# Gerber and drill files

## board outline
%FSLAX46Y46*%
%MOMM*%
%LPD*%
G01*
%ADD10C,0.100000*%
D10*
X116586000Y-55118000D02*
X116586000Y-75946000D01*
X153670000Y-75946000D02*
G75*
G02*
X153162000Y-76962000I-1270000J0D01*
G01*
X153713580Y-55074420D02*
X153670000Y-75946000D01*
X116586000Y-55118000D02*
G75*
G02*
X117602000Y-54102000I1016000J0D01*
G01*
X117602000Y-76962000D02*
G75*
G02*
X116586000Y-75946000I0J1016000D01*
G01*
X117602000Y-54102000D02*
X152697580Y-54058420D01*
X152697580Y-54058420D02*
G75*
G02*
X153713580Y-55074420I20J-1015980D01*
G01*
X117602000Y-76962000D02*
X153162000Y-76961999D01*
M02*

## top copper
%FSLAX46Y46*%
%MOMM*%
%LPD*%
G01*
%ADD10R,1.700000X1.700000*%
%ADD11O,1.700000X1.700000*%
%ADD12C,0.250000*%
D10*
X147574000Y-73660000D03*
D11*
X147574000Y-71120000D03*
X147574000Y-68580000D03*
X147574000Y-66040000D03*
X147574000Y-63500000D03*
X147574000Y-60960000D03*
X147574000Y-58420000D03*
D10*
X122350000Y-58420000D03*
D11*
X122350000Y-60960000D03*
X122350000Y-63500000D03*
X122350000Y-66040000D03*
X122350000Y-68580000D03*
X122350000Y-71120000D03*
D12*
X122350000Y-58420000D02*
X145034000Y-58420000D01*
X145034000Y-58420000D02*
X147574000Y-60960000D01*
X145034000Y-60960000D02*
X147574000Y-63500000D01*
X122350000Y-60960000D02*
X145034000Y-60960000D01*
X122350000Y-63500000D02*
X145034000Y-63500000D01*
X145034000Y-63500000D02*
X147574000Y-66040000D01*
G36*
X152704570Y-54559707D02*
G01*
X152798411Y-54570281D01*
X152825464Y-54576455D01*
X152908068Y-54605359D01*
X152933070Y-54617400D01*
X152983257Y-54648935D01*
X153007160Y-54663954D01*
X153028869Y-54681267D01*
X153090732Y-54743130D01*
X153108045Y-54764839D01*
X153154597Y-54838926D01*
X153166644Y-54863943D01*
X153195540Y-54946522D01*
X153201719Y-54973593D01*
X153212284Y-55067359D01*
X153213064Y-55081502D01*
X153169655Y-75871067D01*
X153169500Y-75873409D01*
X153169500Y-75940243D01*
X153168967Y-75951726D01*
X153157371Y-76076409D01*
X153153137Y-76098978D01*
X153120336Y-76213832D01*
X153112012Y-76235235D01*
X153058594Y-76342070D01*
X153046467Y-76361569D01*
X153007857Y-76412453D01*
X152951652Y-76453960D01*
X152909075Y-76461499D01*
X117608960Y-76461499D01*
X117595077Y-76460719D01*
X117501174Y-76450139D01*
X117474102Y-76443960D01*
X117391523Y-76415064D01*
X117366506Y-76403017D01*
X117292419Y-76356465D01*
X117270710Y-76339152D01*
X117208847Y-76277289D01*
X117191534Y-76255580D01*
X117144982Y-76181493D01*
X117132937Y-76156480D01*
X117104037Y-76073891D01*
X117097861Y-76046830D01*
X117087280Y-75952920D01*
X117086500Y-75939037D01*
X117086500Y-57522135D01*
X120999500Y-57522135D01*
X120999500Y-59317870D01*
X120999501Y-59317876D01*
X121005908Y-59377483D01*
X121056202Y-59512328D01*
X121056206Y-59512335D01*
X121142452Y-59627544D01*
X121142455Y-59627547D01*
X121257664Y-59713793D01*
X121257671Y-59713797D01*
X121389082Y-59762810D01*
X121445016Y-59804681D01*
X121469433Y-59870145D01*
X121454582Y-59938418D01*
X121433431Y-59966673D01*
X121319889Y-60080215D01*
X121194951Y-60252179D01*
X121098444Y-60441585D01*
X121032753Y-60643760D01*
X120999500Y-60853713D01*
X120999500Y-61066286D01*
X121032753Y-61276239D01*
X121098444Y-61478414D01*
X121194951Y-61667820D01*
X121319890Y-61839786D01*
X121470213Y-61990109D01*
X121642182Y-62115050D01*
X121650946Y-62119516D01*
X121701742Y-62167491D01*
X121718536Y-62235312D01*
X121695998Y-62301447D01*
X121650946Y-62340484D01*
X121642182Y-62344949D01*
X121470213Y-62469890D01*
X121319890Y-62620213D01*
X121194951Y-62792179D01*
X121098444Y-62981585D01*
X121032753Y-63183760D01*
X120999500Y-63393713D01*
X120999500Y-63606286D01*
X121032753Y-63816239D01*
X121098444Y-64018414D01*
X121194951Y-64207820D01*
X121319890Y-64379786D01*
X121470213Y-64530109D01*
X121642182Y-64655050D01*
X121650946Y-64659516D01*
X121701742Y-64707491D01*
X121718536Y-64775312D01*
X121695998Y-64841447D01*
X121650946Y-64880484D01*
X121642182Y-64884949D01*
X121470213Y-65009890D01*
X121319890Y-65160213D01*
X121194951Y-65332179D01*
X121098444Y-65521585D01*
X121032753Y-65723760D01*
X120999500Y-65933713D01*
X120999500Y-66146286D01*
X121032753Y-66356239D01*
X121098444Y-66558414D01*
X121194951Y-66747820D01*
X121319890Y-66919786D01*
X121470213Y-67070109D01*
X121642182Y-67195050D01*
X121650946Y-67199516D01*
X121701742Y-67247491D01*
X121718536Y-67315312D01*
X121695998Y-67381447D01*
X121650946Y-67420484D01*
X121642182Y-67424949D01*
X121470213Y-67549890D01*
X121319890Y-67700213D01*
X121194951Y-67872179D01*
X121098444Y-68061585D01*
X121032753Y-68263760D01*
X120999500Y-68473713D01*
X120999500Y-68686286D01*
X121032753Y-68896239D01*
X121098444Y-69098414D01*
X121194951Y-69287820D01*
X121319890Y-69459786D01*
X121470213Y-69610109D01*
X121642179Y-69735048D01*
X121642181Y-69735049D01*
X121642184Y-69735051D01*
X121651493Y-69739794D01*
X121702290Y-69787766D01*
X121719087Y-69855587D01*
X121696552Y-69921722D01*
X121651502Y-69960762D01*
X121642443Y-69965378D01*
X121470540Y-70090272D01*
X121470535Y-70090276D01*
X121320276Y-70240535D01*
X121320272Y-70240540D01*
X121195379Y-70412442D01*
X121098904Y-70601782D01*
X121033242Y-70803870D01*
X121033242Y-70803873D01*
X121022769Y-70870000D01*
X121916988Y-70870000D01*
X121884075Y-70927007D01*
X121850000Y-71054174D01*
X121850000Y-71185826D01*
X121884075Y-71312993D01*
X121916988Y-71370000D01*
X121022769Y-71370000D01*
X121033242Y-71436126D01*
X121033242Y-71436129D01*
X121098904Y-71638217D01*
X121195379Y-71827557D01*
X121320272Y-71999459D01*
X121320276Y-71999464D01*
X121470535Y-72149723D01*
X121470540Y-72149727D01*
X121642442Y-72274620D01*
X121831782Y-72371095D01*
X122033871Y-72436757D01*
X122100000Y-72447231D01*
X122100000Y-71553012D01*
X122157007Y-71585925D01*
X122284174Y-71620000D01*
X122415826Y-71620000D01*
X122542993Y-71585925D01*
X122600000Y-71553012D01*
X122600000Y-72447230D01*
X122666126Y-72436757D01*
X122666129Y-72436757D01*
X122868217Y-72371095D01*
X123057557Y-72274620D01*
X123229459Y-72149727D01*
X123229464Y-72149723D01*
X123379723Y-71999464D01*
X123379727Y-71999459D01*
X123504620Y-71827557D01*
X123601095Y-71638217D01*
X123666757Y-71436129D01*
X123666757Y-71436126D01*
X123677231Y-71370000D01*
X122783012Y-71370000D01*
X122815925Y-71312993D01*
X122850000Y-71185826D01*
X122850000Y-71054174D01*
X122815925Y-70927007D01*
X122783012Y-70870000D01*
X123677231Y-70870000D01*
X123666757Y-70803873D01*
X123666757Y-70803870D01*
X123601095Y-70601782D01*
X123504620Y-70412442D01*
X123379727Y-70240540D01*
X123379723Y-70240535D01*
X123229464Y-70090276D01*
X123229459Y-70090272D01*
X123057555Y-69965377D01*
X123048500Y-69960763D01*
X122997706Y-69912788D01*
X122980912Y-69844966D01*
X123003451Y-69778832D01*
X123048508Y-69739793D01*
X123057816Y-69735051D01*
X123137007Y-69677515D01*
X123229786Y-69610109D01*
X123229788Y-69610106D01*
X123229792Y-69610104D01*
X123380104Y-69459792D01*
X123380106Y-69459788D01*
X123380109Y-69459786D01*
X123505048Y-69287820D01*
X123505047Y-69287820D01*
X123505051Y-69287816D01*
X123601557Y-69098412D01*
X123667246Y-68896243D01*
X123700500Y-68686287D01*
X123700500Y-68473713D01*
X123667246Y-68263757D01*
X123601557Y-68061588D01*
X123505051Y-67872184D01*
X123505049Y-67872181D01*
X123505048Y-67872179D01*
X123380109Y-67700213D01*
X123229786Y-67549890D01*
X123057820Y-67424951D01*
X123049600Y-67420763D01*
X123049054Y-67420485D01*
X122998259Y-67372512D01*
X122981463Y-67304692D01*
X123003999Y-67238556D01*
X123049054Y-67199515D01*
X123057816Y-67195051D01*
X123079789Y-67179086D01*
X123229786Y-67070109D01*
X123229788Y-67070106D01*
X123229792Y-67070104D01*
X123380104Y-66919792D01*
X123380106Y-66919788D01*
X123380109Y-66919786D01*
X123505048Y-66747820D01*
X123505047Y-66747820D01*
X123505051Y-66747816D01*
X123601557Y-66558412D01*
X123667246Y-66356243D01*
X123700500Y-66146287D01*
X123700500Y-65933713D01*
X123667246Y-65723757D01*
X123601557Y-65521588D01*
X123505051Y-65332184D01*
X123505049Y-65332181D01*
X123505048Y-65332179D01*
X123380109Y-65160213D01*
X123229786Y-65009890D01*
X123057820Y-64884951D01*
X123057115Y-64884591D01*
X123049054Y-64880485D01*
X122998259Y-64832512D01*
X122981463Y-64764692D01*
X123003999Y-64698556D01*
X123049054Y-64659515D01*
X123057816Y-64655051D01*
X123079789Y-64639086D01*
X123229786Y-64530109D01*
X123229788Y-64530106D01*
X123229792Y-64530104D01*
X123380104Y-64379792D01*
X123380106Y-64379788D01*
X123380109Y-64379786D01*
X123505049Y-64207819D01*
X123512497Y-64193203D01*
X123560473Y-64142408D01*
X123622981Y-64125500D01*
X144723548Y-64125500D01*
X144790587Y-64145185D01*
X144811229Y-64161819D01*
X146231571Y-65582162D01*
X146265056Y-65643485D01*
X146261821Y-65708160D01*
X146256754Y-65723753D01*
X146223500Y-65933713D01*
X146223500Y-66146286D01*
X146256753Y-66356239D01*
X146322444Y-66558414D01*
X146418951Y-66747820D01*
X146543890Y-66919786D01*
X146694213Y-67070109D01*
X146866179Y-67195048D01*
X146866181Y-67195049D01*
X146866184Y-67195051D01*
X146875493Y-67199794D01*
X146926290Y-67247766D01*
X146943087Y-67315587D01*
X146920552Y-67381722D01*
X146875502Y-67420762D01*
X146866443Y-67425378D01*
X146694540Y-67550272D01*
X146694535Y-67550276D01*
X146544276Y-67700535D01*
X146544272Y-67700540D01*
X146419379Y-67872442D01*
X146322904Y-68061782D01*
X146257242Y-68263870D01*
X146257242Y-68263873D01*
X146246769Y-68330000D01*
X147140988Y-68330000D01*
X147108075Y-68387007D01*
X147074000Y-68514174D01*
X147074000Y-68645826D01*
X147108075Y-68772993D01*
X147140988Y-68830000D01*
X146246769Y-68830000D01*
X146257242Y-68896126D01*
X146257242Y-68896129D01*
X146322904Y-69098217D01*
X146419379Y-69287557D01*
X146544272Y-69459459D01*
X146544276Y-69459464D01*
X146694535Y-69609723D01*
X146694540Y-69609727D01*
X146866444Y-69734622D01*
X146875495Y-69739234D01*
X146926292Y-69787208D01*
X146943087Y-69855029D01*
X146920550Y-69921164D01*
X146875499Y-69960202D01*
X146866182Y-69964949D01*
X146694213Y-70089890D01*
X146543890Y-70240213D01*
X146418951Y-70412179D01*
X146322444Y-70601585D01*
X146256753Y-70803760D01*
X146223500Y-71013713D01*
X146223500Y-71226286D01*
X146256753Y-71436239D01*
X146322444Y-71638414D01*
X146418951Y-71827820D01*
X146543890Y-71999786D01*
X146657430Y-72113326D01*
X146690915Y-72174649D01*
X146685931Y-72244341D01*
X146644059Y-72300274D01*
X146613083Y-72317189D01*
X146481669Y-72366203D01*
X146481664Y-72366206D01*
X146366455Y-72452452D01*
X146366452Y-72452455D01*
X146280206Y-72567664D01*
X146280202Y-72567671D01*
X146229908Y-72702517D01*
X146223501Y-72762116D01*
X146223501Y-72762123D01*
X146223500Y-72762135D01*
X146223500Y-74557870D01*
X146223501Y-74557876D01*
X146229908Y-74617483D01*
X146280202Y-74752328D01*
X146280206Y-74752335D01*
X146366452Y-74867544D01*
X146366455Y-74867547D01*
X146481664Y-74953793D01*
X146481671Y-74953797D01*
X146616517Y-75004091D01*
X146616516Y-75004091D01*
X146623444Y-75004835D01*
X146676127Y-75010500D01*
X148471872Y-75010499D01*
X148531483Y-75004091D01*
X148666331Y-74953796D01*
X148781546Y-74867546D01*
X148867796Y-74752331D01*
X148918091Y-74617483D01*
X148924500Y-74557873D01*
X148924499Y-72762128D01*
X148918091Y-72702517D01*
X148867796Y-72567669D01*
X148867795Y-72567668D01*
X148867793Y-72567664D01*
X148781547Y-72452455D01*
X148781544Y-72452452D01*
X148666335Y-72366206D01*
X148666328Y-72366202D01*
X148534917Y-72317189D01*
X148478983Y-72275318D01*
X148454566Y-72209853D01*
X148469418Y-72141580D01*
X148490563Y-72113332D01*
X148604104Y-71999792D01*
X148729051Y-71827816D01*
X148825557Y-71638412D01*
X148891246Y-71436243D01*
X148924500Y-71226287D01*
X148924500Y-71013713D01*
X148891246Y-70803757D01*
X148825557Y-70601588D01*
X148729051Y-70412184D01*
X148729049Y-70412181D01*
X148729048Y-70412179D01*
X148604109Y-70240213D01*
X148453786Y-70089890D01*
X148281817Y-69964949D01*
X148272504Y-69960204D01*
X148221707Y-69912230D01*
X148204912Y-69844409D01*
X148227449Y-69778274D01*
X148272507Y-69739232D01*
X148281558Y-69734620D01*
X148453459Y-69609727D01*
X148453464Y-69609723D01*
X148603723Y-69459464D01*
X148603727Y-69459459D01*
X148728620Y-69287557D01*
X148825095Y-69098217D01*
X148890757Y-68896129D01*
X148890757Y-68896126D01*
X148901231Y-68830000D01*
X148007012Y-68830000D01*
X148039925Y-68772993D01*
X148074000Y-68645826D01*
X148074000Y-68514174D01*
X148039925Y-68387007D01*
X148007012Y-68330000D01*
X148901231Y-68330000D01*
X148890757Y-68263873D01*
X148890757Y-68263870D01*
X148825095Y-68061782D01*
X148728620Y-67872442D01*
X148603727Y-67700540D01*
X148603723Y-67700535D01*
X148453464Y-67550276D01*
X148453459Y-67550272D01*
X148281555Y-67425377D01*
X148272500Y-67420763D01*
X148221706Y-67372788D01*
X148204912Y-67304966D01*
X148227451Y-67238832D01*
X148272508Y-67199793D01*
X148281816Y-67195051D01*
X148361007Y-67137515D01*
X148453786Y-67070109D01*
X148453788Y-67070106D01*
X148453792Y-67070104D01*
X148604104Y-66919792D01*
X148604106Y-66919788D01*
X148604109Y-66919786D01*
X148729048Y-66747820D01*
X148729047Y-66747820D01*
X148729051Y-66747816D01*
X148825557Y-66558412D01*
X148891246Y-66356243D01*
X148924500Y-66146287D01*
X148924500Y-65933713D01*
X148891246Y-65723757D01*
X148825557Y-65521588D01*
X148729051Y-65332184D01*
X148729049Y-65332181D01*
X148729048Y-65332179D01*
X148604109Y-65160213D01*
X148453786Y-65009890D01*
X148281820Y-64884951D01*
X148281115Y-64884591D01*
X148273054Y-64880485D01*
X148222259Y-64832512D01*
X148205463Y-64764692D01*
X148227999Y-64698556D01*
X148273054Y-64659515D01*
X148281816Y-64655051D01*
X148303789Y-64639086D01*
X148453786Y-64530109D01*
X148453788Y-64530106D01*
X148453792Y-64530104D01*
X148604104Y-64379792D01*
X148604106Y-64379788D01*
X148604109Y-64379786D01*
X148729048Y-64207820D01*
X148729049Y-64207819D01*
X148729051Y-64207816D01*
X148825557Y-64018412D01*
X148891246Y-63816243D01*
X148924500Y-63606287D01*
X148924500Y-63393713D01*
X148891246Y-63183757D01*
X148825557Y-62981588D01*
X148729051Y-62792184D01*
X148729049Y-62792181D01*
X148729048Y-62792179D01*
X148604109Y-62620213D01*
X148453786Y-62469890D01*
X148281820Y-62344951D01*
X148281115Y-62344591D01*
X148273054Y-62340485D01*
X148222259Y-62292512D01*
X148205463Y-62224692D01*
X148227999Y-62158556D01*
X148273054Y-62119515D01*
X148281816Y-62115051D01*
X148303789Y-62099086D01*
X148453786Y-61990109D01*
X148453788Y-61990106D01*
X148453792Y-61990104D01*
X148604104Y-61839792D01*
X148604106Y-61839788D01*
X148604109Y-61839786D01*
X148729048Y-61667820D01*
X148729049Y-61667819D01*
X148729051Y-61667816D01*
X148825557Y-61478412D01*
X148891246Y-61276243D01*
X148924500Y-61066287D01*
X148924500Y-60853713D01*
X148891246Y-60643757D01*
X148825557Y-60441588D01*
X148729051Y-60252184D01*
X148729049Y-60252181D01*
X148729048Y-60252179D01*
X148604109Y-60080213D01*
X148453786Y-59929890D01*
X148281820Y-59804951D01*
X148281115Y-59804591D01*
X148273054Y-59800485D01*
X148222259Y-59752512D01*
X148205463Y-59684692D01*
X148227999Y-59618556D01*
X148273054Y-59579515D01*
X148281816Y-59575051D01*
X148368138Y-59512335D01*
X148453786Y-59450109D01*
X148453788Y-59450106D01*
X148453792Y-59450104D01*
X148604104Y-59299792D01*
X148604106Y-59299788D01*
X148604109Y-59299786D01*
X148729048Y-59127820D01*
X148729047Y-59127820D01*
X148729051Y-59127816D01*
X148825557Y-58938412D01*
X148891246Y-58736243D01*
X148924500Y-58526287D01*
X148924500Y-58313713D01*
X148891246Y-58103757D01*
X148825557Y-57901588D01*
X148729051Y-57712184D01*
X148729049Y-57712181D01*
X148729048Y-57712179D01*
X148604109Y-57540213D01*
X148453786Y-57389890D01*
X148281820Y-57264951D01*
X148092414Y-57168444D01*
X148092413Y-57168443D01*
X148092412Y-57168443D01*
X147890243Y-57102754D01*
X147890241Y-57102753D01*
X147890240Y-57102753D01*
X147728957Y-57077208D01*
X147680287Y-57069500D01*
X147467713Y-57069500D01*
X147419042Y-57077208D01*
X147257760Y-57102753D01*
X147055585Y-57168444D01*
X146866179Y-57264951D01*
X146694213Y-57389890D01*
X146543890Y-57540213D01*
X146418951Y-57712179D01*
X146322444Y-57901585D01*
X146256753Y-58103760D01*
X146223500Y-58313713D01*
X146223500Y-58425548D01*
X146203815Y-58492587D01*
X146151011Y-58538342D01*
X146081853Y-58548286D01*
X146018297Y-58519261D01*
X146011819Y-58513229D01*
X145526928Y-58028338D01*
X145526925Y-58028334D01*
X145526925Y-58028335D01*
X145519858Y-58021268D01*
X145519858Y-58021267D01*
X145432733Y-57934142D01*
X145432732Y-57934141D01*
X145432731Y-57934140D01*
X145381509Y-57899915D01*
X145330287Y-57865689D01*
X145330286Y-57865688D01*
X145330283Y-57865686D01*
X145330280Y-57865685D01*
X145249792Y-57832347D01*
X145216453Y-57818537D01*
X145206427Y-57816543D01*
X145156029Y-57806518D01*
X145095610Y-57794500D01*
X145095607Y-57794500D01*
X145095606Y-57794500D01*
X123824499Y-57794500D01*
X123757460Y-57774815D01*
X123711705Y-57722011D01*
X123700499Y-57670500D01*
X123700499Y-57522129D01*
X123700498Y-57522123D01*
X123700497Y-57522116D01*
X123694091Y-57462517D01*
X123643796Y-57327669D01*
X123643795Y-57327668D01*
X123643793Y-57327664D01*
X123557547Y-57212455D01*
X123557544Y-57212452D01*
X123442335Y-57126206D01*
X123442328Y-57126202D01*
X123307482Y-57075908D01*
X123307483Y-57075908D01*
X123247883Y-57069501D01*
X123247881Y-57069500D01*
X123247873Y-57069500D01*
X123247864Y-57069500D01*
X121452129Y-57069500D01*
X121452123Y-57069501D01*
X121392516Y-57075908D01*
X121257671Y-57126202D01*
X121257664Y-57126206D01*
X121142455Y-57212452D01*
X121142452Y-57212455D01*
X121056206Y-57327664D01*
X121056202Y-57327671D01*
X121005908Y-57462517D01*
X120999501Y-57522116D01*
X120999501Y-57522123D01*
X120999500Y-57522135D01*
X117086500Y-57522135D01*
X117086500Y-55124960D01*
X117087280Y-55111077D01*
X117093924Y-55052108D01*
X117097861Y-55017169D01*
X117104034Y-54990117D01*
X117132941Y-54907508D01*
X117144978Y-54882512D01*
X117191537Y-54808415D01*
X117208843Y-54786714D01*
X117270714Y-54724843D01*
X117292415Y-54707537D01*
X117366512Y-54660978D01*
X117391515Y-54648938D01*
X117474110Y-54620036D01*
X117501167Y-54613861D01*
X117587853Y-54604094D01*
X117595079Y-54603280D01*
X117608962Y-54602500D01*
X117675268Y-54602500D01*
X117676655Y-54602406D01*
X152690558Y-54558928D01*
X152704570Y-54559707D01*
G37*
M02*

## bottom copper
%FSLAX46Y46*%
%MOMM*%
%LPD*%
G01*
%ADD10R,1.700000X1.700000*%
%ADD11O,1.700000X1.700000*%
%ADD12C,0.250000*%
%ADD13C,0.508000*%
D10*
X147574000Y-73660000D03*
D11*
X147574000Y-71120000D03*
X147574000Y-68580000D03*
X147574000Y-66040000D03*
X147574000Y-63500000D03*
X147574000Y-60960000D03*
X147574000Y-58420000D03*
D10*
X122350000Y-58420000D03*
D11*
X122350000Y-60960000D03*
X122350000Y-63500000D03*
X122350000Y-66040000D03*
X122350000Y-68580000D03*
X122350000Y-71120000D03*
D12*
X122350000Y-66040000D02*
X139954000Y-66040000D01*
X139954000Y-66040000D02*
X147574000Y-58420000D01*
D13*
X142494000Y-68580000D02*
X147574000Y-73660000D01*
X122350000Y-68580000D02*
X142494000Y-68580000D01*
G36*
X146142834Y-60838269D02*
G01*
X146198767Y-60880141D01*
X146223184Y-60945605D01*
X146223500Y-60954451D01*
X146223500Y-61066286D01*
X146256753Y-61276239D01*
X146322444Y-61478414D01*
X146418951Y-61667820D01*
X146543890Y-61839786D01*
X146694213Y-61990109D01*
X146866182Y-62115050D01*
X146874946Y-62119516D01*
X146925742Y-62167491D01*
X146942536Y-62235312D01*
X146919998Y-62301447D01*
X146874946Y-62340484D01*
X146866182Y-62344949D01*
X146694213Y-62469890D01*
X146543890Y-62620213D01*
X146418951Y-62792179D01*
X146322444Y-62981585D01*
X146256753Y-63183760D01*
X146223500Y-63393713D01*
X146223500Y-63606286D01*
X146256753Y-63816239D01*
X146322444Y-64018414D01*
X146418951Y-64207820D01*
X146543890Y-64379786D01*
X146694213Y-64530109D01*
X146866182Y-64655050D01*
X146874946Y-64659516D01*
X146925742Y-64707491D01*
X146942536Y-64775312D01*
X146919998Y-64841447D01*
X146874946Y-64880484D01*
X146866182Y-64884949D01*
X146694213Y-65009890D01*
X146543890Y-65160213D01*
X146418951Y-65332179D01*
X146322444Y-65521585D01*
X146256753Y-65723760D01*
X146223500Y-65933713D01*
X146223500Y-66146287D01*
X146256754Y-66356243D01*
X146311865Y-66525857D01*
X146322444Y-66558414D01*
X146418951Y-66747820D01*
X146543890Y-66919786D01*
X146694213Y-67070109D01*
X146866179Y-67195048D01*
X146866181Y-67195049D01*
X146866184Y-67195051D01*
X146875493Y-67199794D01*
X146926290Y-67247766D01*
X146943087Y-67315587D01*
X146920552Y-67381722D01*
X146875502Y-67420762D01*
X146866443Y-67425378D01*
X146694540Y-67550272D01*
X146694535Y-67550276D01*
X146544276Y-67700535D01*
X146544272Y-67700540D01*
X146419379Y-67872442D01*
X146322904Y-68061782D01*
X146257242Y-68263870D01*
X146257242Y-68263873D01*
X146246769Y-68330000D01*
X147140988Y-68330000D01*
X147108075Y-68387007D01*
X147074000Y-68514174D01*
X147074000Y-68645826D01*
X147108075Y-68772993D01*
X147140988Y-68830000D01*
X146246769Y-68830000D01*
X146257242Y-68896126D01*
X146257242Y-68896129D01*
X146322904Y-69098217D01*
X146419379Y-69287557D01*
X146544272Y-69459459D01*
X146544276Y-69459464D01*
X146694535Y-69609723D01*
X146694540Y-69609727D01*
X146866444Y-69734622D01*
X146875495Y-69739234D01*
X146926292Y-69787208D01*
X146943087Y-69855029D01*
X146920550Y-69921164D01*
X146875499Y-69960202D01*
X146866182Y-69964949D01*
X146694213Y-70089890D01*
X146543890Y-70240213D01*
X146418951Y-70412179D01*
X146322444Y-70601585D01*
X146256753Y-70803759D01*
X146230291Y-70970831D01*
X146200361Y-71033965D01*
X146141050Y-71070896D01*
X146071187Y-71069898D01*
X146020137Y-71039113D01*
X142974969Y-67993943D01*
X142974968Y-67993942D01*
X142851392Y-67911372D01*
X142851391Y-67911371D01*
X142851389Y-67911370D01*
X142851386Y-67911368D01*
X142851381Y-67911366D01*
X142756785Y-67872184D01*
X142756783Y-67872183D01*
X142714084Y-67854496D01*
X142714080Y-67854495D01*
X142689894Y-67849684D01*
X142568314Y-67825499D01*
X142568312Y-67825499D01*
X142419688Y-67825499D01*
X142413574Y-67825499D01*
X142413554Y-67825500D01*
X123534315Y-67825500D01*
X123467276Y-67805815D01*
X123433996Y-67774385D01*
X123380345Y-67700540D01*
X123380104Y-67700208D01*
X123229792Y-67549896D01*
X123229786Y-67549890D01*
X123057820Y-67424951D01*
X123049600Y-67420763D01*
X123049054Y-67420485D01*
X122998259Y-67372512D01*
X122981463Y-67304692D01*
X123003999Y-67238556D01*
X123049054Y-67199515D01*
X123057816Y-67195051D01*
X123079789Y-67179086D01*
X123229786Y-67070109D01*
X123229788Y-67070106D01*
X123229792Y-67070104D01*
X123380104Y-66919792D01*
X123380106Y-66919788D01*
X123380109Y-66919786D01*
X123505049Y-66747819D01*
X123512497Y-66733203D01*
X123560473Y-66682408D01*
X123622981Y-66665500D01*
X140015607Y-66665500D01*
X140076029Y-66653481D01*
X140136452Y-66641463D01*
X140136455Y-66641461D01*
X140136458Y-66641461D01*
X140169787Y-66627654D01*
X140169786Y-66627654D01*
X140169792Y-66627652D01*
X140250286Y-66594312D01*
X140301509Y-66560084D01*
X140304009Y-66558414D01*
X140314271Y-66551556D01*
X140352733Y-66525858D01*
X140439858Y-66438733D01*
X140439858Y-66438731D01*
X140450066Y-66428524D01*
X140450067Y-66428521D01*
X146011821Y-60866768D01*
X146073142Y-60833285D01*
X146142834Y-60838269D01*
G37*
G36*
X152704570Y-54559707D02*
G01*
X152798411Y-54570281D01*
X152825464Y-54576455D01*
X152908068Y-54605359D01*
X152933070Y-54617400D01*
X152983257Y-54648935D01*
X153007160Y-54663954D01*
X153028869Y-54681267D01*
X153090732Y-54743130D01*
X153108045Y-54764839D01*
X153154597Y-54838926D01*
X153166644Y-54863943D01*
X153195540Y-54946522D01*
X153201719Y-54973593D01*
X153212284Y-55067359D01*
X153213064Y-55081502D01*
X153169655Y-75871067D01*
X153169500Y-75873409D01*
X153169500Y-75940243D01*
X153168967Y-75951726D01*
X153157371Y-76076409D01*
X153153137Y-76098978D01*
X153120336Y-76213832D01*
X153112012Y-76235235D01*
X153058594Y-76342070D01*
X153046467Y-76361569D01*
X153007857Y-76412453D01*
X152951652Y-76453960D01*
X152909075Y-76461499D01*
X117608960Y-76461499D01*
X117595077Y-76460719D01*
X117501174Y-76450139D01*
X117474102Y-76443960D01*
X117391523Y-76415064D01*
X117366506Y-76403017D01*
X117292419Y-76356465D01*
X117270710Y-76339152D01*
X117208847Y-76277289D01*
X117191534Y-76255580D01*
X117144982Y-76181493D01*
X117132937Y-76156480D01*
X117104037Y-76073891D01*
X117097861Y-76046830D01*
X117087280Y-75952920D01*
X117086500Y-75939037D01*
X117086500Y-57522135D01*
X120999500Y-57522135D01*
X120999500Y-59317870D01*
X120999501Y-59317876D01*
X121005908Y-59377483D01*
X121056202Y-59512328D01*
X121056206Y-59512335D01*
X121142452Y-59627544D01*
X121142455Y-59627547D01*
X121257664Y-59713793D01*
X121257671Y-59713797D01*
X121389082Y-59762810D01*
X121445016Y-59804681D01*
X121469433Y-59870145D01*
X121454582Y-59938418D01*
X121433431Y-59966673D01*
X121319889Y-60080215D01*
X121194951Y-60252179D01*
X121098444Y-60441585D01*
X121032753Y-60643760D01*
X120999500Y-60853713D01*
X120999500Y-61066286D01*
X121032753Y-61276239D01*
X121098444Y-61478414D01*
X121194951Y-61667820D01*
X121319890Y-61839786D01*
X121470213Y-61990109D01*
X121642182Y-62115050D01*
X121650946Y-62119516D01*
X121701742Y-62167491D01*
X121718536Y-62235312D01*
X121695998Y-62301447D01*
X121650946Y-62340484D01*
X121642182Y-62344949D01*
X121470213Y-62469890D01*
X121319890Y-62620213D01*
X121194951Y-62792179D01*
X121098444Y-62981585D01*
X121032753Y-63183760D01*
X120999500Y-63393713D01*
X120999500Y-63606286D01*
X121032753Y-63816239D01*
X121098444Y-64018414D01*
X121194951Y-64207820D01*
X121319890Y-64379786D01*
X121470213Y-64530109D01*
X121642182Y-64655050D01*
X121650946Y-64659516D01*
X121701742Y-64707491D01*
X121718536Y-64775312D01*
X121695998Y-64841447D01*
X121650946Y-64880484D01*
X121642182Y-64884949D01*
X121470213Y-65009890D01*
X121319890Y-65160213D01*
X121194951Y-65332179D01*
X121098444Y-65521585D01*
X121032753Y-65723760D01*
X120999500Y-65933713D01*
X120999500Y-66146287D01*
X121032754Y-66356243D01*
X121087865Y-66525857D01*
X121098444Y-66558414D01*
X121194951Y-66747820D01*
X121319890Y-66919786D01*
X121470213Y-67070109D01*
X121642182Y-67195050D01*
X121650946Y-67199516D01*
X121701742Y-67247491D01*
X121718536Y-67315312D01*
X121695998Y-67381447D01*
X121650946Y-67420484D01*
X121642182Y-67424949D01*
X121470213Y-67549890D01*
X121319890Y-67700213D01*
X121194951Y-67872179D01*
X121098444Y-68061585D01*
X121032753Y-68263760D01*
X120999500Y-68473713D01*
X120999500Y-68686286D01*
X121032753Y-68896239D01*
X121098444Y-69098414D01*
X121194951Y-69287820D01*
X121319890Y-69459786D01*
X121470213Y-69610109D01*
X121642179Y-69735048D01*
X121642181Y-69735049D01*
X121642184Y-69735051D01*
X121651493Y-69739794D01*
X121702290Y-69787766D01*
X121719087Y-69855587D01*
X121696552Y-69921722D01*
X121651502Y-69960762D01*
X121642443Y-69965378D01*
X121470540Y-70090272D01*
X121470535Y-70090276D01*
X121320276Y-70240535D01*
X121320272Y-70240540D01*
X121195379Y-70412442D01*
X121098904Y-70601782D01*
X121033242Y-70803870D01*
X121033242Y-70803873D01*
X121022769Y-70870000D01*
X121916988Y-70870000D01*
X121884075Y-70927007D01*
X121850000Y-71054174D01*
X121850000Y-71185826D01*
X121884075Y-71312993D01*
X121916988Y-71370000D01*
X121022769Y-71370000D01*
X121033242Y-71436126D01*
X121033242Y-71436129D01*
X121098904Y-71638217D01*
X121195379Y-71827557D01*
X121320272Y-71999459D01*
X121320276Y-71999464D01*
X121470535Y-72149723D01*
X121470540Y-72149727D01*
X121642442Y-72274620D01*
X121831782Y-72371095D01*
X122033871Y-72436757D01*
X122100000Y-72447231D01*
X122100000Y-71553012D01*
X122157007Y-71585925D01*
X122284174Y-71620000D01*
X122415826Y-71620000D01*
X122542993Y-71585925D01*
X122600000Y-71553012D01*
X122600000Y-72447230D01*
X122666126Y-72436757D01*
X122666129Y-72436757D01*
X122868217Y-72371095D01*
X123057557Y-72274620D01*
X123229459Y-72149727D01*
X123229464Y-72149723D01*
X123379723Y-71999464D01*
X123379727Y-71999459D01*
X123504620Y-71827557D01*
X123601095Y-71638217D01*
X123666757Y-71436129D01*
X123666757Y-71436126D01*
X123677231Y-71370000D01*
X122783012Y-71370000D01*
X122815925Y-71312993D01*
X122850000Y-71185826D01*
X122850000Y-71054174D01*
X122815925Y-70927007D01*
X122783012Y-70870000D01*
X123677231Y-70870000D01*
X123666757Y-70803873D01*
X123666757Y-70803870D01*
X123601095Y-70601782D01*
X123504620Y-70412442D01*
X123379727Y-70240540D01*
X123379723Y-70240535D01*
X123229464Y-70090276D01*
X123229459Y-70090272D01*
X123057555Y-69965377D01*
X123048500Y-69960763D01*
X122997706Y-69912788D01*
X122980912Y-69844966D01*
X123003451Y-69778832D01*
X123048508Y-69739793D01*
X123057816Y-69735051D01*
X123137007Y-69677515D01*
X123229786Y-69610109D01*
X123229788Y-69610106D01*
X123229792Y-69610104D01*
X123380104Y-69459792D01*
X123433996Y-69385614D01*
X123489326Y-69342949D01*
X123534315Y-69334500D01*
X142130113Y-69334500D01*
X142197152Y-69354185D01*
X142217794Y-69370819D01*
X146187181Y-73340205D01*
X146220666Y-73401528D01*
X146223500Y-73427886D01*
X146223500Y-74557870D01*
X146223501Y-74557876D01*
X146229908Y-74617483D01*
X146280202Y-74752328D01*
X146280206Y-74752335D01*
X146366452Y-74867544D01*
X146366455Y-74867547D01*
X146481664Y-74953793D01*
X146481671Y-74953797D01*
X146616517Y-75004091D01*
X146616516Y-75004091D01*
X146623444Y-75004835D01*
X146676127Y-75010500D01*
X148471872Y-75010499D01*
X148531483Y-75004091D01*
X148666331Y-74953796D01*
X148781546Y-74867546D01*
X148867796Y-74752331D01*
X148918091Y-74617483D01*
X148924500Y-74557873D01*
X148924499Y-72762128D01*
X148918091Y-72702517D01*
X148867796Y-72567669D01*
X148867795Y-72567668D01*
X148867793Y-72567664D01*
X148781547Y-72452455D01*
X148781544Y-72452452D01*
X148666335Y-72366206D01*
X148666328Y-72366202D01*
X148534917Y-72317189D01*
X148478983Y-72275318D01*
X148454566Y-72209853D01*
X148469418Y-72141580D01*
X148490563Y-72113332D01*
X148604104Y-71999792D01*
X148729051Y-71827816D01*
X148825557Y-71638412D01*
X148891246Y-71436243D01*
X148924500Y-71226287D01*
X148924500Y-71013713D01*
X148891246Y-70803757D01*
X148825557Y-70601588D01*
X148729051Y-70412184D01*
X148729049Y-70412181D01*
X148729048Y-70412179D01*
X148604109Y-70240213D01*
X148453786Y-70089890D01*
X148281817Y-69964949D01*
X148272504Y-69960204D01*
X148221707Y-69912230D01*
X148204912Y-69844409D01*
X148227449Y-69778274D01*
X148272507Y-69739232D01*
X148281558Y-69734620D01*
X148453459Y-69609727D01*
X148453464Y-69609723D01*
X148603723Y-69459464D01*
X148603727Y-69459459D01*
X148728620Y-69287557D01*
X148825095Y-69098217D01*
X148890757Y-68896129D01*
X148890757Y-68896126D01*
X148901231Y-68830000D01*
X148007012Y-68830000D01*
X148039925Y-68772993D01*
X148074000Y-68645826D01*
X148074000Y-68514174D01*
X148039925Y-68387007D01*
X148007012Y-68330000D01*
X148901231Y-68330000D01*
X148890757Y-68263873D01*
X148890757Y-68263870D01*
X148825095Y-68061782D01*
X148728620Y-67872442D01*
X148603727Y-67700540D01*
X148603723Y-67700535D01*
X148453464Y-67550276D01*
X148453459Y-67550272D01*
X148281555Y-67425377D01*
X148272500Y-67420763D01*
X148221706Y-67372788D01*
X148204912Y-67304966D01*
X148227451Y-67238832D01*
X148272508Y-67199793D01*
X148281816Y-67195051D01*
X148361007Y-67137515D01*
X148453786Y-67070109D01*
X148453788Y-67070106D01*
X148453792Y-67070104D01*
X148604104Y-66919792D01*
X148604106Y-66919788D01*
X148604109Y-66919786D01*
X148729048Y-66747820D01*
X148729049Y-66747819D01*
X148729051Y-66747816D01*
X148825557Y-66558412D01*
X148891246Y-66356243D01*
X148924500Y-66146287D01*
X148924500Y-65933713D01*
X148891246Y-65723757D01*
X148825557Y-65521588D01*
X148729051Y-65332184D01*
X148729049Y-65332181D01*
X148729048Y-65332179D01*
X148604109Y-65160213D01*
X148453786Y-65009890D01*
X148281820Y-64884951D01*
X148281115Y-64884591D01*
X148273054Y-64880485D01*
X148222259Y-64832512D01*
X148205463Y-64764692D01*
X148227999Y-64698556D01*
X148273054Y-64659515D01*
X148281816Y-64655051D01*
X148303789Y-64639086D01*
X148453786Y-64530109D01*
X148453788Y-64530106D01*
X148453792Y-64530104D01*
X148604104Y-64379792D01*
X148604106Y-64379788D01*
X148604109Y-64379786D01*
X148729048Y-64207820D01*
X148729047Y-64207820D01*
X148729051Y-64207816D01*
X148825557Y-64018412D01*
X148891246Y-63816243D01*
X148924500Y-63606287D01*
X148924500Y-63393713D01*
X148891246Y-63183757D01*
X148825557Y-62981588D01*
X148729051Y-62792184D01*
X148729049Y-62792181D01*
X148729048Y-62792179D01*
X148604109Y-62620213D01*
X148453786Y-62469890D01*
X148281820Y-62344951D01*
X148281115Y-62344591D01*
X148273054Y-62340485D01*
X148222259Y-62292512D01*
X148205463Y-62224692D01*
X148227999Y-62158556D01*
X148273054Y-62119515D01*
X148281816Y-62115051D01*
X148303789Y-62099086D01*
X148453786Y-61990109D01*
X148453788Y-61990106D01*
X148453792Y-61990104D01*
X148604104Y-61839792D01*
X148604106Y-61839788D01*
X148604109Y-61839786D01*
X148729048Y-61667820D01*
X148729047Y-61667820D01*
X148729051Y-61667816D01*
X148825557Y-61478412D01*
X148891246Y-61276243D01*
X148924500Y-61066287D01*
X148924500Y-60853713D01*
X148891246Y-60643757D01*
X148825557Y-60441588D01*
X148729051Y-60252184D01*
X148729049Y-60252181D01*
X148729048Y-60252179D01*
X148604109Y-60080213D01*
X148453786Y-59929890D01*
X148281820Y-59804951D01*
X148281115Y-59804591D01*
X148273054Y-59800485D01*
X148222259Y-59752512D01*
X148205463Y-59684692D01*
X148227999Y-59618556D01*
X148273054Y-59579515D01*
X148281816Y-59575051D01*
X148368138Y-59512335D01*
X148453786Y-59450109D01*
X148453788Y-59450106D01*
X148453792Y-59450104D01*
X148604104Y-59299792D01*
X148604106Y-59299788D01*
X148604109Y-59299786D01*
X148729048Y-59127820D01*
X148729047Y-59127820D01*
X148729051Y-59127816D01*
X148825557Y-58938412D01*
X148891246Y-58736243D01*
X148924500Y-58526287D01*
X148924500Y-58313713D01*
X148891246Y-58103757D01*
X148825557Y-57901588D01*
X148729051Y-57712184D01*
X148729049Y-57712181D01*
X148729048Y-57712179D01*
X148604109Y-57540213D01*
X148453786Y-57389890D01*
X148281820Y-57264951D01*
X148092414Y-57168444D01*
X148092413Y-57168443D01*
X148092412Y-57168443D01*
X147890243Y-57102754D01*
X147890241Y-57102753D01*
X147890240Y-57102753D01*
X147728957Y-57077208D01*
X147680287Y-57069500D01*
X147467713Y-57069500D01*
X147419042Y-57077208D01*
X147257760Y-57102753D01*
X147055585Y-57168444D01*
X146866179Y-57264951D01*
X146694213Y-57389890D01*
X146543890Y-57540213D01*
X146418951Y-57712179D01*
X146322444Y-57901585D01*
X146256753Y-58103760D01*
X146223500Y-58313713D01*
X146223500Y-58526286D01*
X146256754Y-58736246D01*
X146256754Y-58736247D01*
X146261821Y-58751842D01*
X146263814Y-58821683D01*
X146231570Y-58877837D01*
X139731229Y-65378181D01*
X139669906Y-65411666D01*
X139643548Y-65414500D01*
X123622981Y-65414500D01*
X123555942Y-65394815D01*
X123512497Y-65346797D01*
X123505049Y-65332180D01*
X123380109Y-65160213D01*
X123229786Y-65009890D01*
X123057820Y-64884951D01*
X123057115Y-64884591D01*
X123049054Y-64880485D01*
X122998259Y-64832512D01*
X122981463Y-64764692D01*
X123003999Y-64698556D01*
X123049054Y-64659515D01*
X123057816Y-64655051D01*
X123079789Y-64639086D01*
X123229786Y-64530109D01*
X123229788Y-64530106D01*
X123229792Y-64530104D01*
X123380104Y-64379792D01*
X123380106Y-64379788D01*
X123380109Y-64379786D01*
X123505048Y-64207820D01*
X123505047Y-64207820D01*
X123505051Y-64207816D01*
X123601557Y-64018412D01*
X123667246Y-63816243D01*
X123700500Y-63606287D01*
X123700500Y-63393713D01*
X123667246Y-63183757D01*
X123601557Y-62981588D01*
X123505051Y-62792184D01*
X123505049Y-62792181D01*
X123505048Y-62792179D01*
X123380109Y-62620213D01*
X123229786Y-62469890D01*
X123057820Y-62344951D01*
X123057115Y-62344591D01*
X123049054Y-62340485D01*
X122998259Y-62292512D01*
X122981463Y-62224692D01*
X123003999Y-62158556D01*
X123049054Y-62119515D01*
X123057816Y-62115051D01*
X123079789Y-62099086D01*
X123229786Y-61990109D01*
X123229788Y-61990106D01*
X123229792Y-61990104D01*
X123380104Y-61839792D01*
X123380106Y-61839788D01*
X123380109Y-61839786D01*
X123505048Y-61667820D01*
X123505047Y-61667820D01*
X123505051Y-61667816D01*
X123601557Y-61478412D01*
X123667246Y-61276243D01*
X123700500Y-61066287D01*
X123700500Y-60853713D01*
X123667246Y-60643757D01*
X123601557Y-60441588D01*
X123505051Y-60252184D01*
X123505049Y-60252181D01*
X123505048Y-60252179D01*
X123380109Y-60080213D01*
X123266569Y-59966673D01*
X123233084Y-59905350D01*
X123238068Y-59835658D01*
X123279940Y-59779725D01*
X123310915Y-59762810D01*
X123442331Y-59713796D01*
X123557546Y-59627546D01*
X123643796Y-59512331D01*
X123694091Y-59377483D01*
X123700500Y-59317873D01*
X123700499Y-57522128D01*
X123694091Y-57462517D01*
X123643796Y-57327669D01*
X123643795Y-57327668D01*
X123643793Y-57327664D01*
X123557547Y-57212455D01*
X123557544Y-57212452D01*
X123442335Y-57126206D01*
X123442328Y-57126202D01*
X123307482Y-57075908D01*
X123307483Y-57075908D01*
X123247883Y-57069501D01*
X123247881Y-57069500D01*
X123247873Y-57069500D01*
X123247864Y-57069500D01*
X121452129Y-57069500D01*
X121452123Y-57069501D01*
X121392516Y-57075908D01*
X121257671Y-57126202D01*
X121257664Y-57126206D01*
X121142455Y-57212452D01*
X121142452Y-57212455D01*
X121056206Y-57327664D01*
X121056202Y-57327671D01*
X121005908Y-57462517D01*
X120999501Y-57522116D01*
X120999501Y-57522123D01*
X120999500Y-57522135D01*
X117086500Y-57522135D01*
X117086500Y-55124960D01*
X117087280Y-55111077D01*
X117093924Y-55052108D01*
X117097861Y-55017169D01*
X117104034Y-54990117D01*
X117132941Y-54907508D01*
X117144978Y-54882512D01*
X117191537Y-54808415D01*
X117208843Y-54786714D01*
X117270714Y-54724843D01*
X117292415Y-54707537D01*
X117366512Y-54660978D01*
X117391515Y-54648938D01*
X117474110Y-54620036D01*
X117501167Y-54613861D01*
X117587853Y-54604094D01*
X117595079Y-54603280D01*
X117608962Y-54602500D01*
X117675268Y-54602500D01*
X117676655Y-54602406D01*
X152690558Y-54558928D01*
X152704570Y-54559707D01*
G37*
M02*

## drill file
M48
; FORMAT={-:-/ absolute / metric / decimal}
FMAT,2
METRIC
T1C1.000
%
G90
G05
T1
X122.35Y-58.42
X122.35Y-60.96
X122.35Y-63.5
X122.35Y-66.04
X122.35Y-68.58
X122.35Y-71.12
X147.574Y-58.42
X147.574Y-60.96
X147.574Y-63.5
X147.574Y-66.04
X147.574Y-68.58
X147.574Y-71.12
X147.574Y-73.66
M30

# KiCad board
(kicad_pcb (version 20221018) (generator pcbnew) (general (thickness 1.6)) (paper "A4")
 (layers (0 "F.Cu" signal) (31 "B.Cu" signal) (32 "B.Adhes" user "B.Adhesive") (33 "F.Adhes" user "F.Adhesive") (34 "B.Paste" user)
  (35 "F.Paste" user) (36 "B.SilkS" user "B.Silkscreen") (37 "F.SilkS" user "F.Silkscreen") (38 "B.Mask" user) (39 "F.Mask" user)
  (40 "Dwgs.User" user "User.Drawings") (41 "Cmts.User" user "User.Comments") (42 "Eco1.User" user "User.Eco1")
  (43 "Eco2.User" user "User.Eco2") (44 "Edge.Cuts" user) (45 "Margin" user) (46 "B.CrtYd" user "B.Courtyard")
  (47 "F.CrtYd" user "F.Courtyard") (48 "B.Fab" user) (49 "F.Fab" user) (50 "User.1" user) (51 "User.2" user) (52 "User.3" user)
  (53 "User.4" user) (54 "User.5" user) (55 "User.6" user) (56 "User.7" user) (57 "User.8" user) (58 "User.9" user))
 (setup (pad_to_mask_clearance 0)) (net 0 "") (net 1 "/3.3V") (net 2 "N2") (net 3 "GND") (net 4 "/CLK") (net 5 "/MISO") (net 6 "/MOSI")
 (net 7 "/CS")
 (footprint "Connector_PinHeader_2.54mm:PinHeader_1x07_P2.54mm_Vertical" (layer "F.Cu") (at 147.574 73.66 180)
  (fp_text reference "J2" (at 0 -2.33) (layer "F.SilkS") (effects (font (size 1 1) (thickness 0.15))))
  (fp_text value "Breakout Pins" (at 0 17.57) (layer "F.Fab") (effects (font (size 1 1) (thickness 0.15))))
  (pad "1" thru_hole rect (at 0 0 180) (size 1.7 1.7) (drill 1) (layers "*.Cu" "*.Mask") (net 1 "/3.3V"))
  (pad "2" thru_hole oval (at 0 2.54 180) (size 1.7 1.7) (drill 1) (layers "*.Cu" "*.Mask") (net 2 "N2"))
  (pad "3" thru_hole oval (at 0 5.08 180) (size 1.7 1.7) (drill 1) (layers "*.Cu" "*.Mask") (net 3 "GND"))
  (pad "4" thru_hole oval (at 0 7.62 180) (size 1.7 1.7) (drill 1) (layers "*.Cu" "*.Mask") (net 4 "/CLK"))
  (pad "5" thru_hole oval (at 0 10.16 180) (size 1.7 1.7) (drill 1) (layers "*.Cu" "*.Mask") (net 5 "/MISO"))
  (pad "6" thru_hole oval (at 0 12.7 180) (size 1.7 1.7) (drill 1) (layers "*.Cu" "*.Mask") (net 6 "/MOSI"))
  (pad "7" thru_hole oval (at 0 15.24 180) (size 1.7 1.7) (drill 1) (layers "*.Cu" "*.Mask") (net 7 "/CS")))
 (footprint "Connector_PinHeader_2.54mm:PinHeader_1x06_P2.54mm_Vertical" (layer "F.Cu") (at 122.35 58.42)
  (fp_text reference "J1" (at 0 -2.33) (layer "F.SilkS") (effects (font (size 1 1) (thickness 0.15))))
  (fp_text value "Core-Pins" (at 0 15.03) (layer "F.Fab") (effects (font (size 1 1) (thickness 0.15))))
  (pad "1" thru_hole rect (at 0 0) (size 1.7 1.7) (drill 1) (layers "*.Cu" "*.Mask") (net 6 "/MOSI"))
  (pad "2" thru_hole oval (at 0 2.54) (size 1.7 1.7) (drill 1) (layers "*.Cu" "*.Mask") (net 5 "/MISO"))
  (pad "3" thru_hole oval (at 0 5.08) (size 1.7 1.7) (drill 1) (layers "*.Cu" "*.Mask") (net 4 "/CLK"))
  (pad "4" thru_hole oval (at 0 7.62) (size 1.7 1.7) (drill 1) (layers "*.Cu" "*.Mask") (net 7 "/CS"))
  (pad "5" thru_hole oval (at 0 10.16) (size 1.7 1.7) (drill 1) (layers "*.Cu" "*.Mask") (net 1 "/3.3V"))
  (pad "6" thru_hole oval (at 0 12.7) (size 1.7 1.7) (drill 1) (layers "*.Cu" "*.Mask") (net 3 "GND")))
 (gr_line (start 116.586 55.118) (end 116.586 75.946) (stroke (width 0.1) (type default)) (layer "Edge.Cuts"))
 (gr_arc (start 153.67 75.946) (mid 153.535922 76.513961) (end 153.162 76.961999) (stroke (width 0.1) (type default)) (layer "Edge.Cuts"))
 (gr_line (start 153.71358 55.07442) (end 153.67 75.946) (stroke (width 0.1) (type default)) (layer "Edge.Cuts"))
 (gr_arc (start 116.586 55.118) (mid 116.88358 54.39958) (end 117.602 54.102) (stroke (width 0.1) (type default)) (layer "Edge.Cuts"))
 (gr_arc (start 117.602 76.962) (mid 116.88358 76.66442) (end 116.586 75.946) (stroke (width 0.1) (type default)) (layer "Edge.Cuts"))
 (gr_line (start 117.602 54.102) (end 152.69758 54.05842) (stroke (width 0.1) (type default)) (layer "Edge.Cuts"))
 (gr_arc (start 152.69758 54.05842) (mid 153.416 54.356) (end 153.71358 55.07442) (stroke (width 0.1) (type default)) (layer "Edge.Cuts"))
 (gr_line (start 117.602 76.962) (end 153.162 76.961999) (stroke (width 0.1) (type default)) (layer "Edge.Cuts"))
 (segment (start 122.35 58.42) (end 145.034 58.42) (width 0.25) (layer "F.Cu") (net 6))
 (segment (start 145.034 58.42) (end 147.574 60.96) (width 0.25) (layer "F.Cu") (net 6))
 (segment (start 145.034 60.96) (end 147.574 63.5) (width 0.25) (layer "F.Cu") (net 5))
 (segment (start 122.35 60.96) (end 145.034 60.96) (width 0.25) (layer "F.Cu") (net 5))
 (segment (start 122.35 63.5) (end 145.034 63.5) (width 0.25) (layer "F.Cu") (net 4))
 (segment (start 145.034 63.5) (end 147.574 66.04) (width 0.25) (layer "F.Cu") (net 4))
 (segment (start 122.35 66.04) (end 139.954 66.04) (width 0.25) (layer "B.Cu") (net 7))
 (segment (start 139.954 66.04) (end 147.574 58.42) (width 0.25) (layer "B.Cu") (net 7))
 (segment (start 142.494 68.58) (end 147.574 73.66) (width 0.508) (layer "B.Cu") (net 1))
 (segment (start 122.35 68.58) (end 142.494 68.58) (width 0.508) (layer "B.Cu") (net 1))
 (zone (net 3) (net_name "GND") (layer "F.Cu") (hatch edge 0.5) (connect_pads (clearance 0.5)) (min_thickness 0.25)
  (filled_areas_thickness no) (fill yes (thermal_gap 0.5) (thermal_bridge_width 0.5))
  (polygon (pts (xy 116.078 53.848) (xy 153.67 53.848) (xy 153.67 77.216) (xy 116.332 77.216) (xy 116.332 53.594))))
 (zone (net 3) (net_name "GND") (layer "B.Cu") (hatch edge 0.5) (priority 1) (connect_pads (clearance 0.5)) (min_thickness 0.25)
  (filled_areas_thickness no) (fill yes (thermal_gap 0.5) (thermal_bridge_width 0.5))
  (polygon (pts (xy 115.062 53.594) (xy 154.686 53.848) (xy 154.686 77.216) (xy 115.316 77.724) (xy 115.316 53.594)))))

